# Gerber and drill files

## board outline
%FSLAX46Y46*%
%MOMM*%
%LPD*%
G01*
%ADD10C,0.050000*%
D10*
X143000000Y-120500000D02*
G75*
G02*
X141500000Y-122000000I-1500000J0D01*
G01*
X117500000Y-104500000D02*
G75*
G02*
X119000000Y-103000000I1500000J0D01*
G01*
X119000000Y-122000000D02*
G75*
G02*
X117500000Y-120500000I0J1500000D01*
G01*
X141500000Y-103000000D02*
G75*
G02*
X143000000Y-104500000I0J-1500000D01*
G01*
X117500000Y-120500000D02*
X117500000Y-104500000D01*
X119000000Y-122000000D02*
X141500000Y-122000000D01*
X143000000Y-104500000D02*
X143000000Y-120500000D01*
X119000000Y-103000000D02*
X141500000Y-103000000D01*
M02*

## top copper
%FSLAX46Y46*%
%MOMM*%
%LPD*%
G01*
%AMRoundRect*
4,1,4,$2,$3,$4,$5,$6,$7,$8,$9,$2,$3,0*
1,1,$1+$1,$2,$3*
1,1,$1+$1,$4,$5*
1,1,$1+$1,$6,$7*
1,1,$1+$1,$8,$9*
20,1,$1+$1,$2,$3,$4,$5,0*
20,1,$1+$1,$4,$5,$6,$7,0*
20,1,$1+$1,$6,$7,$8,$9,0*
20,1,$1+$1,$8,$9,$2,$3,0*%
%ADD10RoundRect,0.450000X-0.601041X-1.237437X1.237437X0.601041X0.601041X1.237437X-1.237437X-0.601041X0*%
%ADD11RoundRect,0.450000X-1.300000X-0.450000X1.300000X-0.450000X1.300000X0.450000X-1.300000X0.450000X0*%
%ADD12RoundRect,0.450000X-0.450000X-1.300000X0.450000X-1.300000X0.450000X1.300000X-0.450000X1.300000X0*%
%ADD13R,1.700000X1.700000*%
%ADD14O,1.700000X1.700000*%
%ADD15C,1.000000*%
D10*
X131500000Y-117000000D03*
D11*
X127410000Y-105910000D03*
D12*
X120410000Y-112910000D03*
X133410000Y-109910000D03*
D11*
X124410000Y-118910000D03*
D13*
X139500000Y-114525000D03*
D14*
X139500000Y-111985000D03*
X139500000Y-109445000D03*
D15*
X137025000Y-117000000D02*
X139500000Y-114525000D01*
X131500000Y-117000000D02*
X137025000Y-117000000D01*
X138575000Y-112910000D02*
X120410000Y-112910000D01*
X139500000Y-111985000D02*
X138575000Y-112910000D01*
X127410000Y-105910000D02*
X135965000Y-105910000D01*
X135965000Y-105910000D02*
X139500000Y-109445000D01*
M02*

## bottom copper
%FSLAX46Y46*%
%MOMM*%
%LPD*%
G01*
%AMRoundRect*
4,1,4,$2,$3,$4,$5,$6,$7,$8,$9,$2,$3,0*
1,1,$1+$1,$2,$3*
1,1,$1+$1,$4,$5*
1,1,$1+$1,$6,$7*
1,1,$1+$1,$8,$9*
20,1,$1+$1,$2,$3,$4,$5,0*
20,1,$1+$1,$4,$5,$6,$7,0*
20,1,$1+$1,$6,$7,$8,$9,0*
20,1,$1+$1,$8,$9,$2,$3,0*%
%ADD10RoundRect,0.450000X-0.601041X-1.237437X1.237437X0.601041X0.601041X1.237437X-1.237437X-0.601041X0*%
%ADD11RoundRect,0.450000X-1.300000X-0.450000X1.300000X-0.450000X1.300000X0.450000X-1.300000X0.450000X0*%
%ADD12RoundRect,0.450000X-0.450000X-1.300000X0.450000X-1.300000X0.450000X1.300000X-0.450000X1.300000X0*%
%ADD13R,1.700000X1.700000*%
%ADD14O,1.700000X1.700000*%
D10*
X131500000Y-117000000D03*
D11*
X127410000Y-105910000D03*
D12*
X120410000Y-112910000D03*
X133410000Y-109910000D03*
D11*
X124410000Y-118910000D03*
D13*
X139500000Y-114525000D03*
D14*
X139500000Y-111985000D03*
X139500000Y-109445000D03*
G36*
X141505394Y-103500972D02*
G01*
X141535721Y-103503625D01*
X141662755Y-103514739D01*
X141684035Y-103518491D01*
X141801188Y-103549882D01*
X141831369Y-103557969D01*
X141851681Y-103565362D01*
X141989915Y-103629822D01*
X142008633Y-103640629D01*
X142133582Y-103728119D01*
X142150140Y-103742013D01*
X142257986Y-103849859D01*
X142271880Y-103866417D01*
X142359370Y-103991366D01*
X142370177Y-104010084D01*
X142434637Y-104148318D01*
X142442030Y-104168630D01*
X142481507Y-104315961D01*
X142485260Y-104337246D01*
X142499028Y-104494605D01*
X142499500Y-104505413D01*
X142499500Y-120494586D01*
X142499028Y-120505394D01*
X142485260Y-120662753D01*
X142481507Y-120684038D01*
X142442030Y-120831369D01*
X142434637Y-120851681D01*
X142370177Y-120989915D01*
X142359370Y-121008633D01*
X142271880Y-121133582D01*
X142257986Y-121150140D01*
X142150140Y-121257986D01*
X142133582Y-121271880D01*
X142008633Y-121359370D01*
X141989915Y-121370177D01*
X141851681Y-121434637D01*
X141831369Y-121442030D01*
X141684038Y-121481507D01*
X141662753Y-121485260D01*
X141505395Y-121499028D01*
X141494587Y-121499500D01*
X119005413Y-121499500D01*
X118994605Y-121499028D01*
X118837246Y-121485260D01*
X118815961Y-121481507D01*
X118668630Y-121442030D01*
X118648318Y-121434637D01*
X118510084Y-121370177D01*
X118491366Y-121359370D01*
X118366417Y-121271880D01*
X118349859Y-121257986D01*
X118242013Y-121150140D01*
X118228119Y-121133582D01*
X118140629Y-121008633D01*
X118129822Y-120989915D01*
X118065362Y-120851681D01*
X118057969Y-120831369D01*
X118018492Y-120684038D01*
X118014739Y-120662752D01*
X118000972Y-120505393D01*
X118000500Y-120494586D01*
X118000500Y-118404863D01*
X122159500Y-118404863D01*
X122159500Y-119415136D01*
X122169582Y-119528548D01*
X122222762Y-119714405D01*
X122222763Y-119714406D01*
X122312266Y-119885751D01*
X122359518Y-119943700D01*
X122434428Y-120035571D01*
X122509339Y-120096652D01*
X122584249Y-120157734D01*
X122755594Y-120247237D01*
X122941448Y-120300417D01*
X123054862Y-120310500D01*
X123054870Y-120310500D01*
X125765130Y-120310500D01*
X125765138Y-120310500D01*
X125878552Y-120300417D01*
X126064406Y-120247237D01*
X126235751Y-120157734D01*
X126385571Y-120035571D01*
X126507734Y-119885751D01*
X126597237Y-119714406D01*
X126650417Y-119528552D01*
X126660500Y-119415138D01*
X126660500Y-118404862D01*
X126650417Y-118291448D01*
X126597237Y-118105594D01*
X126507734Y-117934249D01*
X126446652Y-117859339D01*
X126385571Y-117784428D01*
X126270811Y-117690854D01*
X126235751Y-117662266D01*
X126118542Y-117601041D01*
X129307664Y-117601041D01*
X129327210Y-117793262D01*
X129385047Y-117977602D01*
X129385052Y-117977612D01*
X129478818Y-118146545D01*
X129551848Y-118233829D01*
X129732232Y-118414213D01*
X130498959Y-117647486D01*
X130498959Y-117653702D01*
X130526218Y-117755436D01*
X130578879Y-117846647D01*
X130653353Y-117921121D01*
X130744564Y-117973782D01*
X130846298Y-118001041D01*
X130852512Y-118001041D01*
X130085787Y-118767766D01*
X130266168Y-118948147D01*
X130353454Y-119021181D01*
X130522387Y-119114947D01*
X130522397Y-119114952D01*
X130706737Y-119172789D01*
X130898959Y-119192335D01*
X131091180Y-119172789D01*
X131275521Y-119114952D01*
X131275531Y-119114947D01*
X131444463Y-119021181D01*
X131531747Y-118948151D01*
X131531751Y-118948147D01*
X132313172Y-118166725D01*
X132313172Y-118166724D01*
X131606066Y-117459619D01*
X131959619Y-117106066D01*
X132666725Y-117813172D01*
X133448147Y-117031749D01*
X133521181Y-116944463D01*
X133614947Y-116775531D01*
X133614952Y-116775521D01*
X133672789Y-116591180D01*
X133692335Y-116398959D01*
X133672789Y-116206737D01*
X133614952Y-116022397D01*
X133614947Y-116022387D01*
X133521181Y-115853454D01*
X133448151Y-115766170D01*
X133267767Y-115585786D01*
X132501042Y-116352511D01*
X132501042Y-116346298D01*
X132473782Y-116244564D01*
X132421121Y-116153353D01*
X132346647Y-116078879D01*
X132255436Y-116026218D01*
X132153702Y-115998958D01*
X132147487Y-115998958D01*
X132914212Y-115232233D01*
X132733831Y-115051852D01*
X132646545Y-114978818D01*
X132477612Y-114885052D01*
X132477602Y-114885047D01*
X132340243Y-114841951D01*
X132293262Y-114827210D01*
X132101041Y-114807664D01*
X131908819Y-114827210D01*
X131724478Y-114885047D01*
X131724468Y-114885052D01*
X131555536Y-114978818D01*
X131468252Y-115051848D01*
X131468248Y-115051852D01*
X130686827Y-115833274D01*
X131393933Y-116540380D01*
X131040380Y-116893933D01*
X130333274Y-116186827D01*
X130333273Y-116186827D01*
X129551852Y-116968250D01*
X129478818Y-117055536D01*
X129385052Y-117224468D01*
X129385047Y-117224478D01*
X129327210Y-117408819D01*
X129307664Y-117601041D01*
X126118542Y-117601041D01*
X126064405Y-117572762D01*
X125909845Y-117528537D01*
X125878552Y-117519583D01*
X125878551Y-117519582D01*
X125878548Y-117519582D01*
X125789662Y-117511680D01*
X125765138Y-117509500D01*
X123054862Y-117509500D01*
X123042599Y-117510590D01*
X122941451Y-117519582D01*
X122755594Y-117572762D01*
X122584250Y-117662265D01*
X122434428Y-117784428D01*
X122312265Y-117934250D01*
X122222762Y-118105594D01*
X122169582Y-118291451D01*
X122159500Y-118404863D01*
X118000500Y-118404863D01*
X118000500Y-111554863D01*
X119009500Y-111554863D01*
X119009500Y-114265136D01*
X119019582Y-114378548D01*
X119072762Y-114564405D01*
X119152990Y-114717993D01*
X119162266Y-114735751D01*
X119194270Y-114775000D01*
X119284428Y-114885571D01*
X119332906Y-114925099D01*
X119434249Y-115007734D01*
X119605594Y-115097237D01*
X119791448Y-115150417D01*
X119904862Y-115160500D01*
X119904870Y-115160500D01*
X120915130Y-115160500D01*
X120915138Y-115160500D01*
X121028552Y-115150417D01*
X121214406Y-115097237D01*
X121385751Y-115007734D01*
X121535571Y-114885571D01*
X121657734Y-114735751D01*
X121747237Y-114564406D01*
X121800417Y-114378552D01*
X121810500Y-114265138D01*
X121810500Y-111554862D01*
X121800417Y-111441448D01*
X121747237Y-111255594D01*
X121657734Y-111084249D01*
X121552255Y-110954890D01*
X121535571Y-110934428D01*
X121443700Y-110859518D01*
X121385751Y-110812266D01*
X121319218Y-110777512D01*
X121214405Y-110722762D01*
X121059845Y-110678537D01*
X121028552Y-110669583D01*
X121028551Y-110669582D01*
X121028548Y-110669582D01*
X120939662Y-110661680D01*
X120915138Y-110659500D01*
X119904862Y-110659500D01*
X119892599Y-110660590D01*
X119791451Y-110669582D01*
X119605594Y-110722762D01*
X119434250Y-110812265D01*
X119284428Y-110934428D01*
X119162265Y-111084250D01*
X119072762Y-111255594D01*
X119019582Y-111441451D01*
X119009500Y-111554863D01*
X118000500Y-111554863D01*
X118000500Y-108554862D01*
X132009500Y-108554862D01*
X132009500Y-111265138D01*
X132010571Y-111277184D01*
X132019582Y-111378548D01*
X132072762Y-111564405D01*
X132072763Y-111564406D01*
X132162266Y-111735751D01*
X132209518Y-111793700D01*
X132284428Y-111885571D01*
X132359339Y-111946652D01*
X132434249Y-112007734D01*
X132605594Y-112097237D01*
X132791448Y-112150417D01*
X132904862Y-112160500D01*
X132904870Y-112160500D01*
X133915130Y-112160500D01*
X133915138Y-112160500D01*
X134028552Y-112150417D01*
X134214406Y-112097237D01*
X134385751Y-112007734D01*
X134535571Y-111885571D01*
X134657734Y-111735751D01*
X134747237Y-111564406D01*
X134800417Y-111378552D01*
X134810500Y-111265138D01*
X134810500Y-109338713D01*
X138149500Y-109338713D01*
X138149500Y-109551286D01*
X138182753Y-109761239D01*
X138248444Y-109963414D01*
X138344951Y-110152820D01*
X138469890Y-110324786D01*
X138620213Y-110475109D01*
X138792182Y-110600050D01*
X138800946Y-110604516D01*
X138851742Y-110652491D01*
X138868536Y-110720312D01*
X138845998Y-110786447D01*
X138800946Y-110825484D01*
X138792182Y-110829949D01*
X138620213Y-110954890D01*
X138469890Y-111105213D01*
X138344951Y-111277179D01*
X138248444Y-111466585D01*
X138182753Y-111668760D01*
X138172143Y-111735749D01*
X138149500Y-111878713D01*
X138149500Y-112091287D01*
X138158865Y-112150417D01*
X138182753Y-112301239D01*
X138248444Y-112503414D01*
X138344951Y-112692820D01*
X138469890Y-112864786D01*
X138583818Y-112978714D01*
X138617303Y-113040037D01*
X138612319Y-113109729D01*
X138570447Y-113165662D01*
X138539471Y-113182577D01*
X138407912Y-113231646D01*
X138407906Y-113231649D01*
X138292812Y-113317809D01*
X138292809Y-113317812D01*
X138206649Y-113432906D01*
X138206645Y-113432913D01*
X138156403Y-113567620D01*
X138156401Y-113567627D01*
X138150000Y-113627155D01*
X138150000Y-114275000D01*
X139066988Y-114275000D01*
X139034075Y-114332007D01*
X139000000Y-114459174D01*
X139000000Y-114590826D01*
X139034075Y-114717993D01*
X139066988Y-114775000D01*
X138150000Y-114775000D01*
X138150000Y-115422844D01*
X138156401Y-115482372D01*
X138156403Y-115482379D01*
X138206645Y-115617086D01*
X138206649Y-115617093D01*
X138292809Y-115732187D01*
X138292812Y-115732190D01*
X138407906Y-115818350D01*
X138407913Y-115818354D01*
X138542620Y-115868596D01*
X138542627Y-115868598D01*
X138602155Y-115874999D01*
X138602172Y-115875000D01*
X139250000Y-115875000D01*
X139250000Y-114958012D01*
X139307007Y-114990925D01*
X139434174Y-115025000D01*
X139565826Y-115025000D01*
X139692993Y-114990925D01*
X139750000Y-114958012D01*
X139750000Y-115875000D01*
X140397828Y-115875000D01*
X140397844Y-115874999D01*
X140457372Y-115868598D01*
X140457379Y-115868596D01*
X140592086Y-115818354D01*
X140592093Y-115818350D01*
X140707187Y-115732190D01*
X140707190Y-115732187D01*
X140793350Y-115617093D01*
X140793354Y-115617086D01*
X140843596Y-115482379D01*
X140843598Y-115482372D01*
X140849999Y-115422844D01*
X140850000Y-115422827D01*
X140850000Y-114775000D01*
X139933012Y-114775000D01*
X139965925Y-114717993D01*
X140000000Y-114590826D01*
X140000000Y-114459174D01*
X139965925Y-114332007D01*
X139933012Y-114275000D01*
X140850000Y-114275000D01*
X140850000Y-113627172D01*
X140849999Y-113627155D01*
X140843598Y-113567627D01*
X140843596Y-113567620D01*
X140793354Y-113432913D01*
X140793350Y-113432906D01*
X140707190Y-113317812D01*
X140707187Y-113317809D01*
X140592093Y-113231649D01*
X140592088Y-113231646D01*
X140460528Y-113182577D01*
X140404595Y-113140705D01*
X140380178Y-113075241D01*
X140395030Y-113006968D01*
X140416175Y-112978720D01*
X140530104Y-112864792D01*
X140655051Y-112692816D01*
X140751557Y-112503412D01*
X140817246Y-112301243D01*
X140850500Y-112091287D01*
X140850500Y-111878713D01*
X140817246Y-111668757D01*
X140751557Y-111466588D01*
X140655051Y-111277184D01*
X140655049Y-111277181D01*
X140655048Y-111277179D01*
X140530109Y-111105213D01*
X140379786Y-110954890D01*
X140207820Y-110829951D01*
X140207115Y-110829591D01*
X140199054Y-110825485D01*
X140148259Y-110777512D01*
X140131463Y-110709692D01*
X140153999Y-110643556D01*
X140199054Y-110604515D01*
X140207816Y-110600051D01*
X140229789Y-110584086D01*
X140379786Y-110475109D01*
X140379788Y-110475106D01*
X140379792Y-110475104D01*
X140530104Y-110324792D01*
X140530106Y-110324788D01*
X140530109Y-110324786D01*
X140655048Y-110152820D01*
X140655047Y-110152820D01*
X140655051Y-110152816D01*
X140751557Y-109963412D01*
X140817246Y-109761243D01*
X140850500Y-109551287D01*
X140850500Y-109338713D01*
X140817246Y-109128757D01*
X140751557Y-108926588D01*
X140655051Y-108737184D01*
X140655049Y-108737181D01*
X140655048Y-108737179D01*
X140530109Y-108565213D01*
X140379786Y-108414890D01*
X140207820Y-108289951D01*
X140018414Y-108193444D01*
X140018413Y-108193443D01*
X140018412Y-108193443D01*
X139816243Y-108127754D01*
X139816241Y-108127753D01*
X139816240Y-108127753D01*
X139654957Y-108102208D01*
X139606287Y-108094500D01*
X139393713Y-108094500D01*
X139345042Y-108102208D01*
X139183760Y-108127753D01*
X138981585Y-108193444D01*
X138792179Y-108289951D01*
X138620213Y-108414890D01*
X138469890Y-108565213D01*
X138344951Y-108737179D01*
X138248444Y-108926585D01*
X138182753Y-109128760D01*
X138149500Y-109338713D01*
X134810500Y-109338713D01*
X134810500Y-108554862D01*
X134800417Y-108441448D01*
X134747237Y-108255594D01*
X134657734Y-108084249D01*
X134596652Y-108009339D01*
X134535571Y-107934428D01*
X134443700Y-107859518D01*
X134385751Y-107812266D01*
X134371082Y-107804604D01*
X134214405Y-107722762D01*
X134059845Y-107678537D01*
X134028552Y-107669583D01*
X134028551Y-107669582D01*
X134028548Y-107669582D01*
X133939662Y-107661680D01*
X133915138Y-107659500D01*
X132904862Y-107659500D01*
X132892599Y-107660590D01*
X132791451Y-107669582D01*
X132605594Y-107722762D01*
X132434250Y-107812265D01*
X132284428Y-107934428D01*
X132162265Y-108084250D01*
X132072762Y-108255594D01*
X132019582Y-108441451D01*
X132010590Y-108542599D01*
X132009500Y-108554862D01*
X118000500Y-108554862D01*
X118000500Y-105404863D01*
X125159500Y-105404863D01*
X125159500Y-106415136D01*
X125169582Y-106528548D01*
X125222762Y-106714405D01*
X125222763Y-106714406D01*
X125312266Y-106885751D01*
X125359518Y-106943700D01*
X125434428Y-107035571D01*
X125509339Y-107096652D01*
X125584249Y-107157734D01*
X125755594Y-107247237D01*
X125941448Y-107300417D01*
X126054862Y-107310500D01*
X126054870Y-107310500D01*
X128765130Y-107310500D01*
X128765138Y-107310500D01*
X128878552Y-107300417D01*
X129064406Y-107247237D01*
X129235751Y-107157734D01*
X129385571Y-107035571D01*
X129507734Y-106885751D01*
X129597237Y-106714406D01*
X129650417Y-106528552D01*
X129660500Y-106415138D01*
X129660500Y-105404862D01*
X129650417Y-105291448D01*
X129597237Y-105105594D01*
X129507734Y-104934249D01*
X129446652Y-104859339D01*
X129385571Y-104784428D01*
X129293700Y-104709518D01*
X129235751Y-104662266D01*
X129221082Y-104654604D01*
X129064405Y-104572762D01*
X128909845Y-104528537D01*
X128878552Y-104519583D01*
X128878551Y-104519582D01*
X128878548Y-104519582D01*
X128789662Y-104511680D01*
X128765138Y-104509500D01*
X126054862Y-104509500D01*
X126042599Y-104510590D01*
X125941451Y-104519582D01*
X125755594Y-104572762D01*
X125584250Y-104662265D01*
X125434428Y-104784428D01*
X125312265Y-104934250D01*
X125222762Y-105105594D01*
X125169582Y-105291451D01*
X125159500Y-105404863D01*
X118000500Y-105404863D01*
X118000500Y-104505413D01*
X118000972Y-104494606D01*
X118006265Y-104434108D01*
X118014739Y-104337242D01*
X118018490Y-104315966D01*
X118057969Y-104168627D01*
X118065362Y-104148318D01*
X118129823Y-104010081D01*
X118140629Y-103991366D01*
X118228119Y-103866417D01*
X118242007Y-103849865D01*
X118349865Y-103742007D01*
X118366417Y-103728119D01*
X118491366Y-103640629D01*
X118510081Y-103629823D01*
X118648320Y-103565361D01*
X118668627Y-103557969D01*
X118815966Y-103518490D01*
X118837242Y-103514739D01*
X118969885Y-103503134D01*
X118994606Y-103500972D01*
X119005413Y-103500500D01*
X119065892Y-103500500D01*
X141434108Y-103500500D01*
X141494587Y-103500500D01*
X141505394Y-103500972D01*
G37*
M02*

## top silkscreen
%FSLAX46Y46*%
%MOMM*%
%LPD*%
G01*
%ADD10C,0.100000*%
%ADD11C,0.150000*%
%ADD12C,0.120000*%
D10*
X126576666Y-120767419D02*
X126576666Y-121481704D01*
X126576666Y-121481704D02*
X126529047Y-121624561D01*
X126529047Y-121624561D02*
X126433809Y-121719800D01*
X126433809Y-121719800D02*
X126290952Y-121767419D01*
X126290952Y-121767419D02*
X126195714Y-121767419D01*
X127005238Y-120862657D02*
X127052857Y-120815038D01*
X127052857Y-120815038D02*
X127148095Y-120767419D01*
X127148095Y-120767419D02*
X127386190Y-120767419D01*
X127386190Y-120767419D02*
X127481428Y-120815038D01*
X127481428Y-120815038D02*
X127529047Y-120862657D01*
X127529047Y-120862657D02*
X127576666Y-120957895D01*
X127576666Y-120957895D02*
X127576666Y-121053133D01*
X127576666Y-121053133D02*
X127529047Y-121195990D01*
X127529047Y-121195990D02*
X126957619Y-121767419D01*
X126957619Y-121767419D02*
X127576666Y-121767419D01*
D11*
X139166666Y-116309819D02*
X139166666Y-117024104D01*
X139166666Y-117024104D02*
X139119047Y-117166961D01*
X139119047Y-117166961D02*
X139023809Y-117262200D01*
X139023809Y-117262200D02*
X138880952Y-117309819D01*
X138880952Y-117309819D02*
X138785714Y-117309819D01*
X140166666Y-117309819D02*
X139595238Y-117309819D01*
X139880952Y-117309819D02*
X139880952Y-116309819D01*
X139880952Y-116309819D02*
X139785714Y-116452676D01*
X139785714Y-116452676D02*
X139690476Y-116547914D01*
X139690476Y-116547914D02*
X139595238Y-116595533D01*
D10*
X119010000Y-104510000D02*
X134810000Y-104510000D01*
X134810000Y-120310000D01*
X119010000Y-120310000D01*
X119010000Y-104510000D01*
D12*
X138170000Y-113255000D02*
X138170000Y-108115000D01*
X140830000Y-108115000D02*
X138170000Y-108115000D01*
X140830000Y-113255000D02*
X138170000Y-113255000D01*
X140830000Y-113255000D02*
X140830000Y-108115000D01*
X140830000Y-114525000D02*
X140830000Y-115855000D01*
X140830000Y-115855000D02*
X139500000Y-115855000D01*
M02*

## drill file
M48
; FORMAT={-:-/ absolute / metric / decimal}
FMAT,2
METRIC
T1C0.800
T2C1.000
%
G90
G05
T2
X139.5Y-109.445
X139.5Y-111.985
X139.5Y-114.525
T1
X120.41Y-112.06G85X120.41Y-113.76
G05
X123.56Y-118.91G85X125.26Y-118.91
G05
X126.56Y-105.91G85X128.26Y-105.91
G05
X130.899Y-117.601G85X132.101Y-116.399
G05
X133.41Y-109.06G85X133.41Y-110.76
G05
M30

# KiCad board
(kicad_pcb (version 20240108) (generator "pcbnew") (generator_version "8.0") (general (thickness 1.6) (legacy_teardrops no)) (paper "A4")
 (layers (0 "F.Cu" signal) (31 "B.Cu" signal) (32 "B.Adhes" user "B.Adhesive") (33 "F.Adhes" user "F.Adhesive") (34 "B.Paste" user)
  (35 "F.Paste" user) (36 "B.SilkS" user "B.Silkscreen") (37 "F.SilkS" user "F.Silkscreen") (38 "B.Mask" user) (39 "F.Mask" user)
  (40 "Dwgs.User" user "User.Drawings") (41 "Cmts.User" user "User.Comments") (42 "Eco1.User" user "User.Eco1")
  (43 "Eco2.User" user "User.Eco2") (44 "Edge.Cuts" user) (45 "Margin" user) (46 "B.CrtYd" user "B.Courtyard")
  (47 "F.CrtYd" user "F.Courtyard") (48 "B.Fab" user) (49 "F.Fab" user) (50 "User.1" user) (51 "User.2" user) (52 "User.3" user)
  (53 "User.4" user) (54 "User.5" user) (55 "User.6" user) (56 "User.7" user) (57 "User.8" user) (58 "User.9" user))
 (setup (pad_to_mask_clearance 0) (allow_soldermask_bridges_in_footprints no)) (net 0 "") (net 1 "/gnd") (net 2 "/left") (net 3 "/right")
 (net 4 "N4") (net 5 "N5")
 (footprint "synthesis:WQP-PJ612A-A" (layer "F.Cu") (at 126.91 112.41)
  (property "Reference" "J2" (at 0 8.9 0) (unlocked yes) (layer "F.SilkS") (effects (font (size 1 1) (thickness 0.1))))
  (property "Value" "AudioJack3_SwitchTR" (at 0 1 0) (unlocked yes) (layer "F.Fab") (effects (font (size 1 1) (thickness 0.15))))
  (fp_rect (start -7.9 -7.9) (end 7.9 7.9) (stroke (width 0.1) (type default)) (fill none) (layer "F.SilkS"))
  (pad "1" thru_hole roundrect (at 4.59 4.59 45) (size 3.5 1.8) (drill oval 2.5 0.8) (layers "*.Cu" "*.Mask") (remove_unused_layers no)
   (roundrect_rratio 0.25) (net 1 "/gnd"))
  (pad "2" thru_hole roundrect (at 0.5 -6.5) (size 3.5 1.8) (drill oval 2.5 0.8) (layers "*.Cu" "*.Mask") (remove_unused_layers no)
   (roundrect_rratio 0.25) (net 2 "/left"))
  (pad "3" thru_hole roundrect (at -6.5 0.5) (size 1.8 3.5) (drill oval 0.8 2.5) (layers "*.Cu" "*.Mask") (remove_unused_layers no)
   (roundrect_rratio 0.25) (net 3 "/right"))
  (pad "4" thru_hole roundrect (at 6.5 -2.5) (size 1.8 3.5) (drill oval 0.8 2.5) (layers "*.Cu" "*.Mask") (remove_unused_layers no)
   (roundrect_rratio 0.25) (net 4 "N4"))
  (pad "5" thru_hole roundrect (at -2.5 6.5) (size 3.5 1.8) (drill oval 2.5 0.8) (layers "*.Cu" "*.Mask") (remove_unused_layers no)
   (roundrect_rratio 0.25) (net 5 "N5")))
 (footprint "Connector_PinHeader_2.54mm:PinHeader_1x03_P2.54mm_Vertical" (layer "F.Cu") (at 139.5 114.525 180)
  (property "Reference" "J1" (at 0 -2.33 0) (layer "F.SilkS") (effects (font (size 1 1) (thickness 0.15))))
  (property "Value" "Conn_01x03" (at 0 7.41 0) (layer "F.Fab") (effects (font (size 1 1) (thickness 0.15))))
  (fp_line (start 1.33 1.27) (end 1.33 6.41) (stroke (width 0.12) (type solid)) (layer "F.SilkS"))
  (fp_line (start -1.33 6.41) (end 1.33 6.41) (stroke (width 0.12) (type solid)) (layer "F.SilkS"))
  (fp_line (start -1.33 1.27) (end 1.33 1.27) (stroke (width 0.12) (type solid)) (layer "F.SilkS"))
  (fp_line (start -1.33 1.27) (end -1.33 6.41) (stroke (width 0.12) (type solid)) (layer "F.SilkS"))
  (fp_line (start -1.33 0) (end -1.33 -1.33) (stroke (width 0.12) (type solid)) (layer "F.SilkS"))
  (fp_line (start -1.33 -1.33) (end 0 -1.33) (stroke (width 0.12) (type solid)) (layer "F.SilkS"))
  (pad "1" thru_hole rect (at 0 0 180) (size 1.7 1.7) (drill 1) (layers "*.Cu" "*.Mask") (remove_unused_layers no) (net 1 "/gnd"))
  (pad "2" thru_hole oval (at 0 2.54 180) (size 1.7 1.7) (drill 1) (layers "*.Cu" "*.Mask") (remove_unused_layers no) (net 3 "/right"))
  (pad "3" thru_hole oval (at 0 5.08 180) (size 1.7 1.7) (drill 1) (layers "*.Cu" "*.Mask") (remove_unused_layers no) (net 2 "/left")))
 (gr_arc (start 143 120.5) (mid 142.56066 121.56066) (end 141.5 122) (stroke (width 0.05) (type default)) (layer "Edge.Cuts"))
 (gr_arc (start 117.5 104.5) (mid 117.93934 103.43934) (end 119 103) (stroke (width 0.05) (type default)) (layer "Edge.Cuts"))
 (gr_arc (start 119 122) (mid 117.93934 121.56066) (end 117.5 120.5) (stroke (width 0.05) (type default)) (layer "Edge.Cuts"))
 (gr_arc (start 141.5 103) (mid 142.56066 103.43934) (end 143 104.5) (stroke (width 0.05) (type default)) (layer "Edge.Cuts"))
 (gr_line (start 117.5 120.5) (end 117.5 104.5) (stroke (width 0.05) (type default)) (layer "Edge.Cuts"))
 (gr_line (start 119 122) (end 141.5 122) (stroke (width 0.05) (type default)) (layer "Edge.Cuts"))
 (gr_line (start 143 104.5) (end 143 120.5) (stroke (width 0.05) (type default)) (layer "Edge.Cuts"))
 (gr_line (start 119 103) (end 141.5 103) (stroke (width 0.05) (type default)) (layer "Edge.Cuts"))
 (segment (start 137.025 117) (end 139.5 114.525) (width 1) (layer "F.Cu") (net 1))
 (segment (start 131.5 117) (end 137.025 117) (width 1) (layer "F.Cu") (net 1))
 (segment (start 138.575 112.91) (end 120.41 112.91) (width 1) (layer "F.Cu") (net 3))
 (segment (start 139.5 111.985) (end 138.575 112.91) (width 1) (layer "F.Cu") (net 3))
 (segment (start 127.41 105.91) (end 135.965 105.91) (width 1) (layer "F.Cu") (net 2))
 (segment (start 135.965 105.91) (end 139.5 109.445) (width 1) (layer "F.Cu") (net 2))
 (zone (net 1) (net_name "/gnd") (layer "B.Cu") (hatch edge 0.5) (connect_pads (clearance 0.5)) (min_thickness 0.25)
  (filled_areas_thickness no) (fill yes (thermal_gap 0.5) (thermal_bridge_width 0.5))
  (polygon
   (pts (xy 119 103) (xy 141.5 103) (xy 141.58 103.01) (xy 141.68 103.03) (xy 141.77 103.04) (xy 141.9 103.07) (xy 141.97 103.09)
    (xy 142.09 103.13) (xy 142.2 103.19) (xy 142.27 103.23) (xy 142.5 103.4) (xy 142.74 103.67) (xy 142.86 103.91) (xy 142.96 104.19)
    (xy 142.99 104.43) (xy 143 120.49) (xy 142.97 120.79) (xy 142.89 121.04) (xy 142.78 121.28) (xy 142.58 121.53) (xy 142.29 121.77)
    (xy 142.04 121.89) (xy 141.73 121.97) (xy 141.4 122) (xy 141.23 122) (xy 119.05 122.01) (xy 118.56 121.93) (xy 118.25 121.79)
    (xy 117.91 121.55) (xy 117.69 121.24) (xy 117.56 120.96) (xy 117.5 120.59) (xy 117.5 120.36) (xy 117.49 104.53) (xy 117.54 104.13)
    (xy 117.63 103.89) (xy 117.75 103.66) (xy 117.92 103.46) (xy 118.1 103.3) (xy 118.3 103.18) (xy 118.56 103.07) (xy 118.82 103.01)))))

